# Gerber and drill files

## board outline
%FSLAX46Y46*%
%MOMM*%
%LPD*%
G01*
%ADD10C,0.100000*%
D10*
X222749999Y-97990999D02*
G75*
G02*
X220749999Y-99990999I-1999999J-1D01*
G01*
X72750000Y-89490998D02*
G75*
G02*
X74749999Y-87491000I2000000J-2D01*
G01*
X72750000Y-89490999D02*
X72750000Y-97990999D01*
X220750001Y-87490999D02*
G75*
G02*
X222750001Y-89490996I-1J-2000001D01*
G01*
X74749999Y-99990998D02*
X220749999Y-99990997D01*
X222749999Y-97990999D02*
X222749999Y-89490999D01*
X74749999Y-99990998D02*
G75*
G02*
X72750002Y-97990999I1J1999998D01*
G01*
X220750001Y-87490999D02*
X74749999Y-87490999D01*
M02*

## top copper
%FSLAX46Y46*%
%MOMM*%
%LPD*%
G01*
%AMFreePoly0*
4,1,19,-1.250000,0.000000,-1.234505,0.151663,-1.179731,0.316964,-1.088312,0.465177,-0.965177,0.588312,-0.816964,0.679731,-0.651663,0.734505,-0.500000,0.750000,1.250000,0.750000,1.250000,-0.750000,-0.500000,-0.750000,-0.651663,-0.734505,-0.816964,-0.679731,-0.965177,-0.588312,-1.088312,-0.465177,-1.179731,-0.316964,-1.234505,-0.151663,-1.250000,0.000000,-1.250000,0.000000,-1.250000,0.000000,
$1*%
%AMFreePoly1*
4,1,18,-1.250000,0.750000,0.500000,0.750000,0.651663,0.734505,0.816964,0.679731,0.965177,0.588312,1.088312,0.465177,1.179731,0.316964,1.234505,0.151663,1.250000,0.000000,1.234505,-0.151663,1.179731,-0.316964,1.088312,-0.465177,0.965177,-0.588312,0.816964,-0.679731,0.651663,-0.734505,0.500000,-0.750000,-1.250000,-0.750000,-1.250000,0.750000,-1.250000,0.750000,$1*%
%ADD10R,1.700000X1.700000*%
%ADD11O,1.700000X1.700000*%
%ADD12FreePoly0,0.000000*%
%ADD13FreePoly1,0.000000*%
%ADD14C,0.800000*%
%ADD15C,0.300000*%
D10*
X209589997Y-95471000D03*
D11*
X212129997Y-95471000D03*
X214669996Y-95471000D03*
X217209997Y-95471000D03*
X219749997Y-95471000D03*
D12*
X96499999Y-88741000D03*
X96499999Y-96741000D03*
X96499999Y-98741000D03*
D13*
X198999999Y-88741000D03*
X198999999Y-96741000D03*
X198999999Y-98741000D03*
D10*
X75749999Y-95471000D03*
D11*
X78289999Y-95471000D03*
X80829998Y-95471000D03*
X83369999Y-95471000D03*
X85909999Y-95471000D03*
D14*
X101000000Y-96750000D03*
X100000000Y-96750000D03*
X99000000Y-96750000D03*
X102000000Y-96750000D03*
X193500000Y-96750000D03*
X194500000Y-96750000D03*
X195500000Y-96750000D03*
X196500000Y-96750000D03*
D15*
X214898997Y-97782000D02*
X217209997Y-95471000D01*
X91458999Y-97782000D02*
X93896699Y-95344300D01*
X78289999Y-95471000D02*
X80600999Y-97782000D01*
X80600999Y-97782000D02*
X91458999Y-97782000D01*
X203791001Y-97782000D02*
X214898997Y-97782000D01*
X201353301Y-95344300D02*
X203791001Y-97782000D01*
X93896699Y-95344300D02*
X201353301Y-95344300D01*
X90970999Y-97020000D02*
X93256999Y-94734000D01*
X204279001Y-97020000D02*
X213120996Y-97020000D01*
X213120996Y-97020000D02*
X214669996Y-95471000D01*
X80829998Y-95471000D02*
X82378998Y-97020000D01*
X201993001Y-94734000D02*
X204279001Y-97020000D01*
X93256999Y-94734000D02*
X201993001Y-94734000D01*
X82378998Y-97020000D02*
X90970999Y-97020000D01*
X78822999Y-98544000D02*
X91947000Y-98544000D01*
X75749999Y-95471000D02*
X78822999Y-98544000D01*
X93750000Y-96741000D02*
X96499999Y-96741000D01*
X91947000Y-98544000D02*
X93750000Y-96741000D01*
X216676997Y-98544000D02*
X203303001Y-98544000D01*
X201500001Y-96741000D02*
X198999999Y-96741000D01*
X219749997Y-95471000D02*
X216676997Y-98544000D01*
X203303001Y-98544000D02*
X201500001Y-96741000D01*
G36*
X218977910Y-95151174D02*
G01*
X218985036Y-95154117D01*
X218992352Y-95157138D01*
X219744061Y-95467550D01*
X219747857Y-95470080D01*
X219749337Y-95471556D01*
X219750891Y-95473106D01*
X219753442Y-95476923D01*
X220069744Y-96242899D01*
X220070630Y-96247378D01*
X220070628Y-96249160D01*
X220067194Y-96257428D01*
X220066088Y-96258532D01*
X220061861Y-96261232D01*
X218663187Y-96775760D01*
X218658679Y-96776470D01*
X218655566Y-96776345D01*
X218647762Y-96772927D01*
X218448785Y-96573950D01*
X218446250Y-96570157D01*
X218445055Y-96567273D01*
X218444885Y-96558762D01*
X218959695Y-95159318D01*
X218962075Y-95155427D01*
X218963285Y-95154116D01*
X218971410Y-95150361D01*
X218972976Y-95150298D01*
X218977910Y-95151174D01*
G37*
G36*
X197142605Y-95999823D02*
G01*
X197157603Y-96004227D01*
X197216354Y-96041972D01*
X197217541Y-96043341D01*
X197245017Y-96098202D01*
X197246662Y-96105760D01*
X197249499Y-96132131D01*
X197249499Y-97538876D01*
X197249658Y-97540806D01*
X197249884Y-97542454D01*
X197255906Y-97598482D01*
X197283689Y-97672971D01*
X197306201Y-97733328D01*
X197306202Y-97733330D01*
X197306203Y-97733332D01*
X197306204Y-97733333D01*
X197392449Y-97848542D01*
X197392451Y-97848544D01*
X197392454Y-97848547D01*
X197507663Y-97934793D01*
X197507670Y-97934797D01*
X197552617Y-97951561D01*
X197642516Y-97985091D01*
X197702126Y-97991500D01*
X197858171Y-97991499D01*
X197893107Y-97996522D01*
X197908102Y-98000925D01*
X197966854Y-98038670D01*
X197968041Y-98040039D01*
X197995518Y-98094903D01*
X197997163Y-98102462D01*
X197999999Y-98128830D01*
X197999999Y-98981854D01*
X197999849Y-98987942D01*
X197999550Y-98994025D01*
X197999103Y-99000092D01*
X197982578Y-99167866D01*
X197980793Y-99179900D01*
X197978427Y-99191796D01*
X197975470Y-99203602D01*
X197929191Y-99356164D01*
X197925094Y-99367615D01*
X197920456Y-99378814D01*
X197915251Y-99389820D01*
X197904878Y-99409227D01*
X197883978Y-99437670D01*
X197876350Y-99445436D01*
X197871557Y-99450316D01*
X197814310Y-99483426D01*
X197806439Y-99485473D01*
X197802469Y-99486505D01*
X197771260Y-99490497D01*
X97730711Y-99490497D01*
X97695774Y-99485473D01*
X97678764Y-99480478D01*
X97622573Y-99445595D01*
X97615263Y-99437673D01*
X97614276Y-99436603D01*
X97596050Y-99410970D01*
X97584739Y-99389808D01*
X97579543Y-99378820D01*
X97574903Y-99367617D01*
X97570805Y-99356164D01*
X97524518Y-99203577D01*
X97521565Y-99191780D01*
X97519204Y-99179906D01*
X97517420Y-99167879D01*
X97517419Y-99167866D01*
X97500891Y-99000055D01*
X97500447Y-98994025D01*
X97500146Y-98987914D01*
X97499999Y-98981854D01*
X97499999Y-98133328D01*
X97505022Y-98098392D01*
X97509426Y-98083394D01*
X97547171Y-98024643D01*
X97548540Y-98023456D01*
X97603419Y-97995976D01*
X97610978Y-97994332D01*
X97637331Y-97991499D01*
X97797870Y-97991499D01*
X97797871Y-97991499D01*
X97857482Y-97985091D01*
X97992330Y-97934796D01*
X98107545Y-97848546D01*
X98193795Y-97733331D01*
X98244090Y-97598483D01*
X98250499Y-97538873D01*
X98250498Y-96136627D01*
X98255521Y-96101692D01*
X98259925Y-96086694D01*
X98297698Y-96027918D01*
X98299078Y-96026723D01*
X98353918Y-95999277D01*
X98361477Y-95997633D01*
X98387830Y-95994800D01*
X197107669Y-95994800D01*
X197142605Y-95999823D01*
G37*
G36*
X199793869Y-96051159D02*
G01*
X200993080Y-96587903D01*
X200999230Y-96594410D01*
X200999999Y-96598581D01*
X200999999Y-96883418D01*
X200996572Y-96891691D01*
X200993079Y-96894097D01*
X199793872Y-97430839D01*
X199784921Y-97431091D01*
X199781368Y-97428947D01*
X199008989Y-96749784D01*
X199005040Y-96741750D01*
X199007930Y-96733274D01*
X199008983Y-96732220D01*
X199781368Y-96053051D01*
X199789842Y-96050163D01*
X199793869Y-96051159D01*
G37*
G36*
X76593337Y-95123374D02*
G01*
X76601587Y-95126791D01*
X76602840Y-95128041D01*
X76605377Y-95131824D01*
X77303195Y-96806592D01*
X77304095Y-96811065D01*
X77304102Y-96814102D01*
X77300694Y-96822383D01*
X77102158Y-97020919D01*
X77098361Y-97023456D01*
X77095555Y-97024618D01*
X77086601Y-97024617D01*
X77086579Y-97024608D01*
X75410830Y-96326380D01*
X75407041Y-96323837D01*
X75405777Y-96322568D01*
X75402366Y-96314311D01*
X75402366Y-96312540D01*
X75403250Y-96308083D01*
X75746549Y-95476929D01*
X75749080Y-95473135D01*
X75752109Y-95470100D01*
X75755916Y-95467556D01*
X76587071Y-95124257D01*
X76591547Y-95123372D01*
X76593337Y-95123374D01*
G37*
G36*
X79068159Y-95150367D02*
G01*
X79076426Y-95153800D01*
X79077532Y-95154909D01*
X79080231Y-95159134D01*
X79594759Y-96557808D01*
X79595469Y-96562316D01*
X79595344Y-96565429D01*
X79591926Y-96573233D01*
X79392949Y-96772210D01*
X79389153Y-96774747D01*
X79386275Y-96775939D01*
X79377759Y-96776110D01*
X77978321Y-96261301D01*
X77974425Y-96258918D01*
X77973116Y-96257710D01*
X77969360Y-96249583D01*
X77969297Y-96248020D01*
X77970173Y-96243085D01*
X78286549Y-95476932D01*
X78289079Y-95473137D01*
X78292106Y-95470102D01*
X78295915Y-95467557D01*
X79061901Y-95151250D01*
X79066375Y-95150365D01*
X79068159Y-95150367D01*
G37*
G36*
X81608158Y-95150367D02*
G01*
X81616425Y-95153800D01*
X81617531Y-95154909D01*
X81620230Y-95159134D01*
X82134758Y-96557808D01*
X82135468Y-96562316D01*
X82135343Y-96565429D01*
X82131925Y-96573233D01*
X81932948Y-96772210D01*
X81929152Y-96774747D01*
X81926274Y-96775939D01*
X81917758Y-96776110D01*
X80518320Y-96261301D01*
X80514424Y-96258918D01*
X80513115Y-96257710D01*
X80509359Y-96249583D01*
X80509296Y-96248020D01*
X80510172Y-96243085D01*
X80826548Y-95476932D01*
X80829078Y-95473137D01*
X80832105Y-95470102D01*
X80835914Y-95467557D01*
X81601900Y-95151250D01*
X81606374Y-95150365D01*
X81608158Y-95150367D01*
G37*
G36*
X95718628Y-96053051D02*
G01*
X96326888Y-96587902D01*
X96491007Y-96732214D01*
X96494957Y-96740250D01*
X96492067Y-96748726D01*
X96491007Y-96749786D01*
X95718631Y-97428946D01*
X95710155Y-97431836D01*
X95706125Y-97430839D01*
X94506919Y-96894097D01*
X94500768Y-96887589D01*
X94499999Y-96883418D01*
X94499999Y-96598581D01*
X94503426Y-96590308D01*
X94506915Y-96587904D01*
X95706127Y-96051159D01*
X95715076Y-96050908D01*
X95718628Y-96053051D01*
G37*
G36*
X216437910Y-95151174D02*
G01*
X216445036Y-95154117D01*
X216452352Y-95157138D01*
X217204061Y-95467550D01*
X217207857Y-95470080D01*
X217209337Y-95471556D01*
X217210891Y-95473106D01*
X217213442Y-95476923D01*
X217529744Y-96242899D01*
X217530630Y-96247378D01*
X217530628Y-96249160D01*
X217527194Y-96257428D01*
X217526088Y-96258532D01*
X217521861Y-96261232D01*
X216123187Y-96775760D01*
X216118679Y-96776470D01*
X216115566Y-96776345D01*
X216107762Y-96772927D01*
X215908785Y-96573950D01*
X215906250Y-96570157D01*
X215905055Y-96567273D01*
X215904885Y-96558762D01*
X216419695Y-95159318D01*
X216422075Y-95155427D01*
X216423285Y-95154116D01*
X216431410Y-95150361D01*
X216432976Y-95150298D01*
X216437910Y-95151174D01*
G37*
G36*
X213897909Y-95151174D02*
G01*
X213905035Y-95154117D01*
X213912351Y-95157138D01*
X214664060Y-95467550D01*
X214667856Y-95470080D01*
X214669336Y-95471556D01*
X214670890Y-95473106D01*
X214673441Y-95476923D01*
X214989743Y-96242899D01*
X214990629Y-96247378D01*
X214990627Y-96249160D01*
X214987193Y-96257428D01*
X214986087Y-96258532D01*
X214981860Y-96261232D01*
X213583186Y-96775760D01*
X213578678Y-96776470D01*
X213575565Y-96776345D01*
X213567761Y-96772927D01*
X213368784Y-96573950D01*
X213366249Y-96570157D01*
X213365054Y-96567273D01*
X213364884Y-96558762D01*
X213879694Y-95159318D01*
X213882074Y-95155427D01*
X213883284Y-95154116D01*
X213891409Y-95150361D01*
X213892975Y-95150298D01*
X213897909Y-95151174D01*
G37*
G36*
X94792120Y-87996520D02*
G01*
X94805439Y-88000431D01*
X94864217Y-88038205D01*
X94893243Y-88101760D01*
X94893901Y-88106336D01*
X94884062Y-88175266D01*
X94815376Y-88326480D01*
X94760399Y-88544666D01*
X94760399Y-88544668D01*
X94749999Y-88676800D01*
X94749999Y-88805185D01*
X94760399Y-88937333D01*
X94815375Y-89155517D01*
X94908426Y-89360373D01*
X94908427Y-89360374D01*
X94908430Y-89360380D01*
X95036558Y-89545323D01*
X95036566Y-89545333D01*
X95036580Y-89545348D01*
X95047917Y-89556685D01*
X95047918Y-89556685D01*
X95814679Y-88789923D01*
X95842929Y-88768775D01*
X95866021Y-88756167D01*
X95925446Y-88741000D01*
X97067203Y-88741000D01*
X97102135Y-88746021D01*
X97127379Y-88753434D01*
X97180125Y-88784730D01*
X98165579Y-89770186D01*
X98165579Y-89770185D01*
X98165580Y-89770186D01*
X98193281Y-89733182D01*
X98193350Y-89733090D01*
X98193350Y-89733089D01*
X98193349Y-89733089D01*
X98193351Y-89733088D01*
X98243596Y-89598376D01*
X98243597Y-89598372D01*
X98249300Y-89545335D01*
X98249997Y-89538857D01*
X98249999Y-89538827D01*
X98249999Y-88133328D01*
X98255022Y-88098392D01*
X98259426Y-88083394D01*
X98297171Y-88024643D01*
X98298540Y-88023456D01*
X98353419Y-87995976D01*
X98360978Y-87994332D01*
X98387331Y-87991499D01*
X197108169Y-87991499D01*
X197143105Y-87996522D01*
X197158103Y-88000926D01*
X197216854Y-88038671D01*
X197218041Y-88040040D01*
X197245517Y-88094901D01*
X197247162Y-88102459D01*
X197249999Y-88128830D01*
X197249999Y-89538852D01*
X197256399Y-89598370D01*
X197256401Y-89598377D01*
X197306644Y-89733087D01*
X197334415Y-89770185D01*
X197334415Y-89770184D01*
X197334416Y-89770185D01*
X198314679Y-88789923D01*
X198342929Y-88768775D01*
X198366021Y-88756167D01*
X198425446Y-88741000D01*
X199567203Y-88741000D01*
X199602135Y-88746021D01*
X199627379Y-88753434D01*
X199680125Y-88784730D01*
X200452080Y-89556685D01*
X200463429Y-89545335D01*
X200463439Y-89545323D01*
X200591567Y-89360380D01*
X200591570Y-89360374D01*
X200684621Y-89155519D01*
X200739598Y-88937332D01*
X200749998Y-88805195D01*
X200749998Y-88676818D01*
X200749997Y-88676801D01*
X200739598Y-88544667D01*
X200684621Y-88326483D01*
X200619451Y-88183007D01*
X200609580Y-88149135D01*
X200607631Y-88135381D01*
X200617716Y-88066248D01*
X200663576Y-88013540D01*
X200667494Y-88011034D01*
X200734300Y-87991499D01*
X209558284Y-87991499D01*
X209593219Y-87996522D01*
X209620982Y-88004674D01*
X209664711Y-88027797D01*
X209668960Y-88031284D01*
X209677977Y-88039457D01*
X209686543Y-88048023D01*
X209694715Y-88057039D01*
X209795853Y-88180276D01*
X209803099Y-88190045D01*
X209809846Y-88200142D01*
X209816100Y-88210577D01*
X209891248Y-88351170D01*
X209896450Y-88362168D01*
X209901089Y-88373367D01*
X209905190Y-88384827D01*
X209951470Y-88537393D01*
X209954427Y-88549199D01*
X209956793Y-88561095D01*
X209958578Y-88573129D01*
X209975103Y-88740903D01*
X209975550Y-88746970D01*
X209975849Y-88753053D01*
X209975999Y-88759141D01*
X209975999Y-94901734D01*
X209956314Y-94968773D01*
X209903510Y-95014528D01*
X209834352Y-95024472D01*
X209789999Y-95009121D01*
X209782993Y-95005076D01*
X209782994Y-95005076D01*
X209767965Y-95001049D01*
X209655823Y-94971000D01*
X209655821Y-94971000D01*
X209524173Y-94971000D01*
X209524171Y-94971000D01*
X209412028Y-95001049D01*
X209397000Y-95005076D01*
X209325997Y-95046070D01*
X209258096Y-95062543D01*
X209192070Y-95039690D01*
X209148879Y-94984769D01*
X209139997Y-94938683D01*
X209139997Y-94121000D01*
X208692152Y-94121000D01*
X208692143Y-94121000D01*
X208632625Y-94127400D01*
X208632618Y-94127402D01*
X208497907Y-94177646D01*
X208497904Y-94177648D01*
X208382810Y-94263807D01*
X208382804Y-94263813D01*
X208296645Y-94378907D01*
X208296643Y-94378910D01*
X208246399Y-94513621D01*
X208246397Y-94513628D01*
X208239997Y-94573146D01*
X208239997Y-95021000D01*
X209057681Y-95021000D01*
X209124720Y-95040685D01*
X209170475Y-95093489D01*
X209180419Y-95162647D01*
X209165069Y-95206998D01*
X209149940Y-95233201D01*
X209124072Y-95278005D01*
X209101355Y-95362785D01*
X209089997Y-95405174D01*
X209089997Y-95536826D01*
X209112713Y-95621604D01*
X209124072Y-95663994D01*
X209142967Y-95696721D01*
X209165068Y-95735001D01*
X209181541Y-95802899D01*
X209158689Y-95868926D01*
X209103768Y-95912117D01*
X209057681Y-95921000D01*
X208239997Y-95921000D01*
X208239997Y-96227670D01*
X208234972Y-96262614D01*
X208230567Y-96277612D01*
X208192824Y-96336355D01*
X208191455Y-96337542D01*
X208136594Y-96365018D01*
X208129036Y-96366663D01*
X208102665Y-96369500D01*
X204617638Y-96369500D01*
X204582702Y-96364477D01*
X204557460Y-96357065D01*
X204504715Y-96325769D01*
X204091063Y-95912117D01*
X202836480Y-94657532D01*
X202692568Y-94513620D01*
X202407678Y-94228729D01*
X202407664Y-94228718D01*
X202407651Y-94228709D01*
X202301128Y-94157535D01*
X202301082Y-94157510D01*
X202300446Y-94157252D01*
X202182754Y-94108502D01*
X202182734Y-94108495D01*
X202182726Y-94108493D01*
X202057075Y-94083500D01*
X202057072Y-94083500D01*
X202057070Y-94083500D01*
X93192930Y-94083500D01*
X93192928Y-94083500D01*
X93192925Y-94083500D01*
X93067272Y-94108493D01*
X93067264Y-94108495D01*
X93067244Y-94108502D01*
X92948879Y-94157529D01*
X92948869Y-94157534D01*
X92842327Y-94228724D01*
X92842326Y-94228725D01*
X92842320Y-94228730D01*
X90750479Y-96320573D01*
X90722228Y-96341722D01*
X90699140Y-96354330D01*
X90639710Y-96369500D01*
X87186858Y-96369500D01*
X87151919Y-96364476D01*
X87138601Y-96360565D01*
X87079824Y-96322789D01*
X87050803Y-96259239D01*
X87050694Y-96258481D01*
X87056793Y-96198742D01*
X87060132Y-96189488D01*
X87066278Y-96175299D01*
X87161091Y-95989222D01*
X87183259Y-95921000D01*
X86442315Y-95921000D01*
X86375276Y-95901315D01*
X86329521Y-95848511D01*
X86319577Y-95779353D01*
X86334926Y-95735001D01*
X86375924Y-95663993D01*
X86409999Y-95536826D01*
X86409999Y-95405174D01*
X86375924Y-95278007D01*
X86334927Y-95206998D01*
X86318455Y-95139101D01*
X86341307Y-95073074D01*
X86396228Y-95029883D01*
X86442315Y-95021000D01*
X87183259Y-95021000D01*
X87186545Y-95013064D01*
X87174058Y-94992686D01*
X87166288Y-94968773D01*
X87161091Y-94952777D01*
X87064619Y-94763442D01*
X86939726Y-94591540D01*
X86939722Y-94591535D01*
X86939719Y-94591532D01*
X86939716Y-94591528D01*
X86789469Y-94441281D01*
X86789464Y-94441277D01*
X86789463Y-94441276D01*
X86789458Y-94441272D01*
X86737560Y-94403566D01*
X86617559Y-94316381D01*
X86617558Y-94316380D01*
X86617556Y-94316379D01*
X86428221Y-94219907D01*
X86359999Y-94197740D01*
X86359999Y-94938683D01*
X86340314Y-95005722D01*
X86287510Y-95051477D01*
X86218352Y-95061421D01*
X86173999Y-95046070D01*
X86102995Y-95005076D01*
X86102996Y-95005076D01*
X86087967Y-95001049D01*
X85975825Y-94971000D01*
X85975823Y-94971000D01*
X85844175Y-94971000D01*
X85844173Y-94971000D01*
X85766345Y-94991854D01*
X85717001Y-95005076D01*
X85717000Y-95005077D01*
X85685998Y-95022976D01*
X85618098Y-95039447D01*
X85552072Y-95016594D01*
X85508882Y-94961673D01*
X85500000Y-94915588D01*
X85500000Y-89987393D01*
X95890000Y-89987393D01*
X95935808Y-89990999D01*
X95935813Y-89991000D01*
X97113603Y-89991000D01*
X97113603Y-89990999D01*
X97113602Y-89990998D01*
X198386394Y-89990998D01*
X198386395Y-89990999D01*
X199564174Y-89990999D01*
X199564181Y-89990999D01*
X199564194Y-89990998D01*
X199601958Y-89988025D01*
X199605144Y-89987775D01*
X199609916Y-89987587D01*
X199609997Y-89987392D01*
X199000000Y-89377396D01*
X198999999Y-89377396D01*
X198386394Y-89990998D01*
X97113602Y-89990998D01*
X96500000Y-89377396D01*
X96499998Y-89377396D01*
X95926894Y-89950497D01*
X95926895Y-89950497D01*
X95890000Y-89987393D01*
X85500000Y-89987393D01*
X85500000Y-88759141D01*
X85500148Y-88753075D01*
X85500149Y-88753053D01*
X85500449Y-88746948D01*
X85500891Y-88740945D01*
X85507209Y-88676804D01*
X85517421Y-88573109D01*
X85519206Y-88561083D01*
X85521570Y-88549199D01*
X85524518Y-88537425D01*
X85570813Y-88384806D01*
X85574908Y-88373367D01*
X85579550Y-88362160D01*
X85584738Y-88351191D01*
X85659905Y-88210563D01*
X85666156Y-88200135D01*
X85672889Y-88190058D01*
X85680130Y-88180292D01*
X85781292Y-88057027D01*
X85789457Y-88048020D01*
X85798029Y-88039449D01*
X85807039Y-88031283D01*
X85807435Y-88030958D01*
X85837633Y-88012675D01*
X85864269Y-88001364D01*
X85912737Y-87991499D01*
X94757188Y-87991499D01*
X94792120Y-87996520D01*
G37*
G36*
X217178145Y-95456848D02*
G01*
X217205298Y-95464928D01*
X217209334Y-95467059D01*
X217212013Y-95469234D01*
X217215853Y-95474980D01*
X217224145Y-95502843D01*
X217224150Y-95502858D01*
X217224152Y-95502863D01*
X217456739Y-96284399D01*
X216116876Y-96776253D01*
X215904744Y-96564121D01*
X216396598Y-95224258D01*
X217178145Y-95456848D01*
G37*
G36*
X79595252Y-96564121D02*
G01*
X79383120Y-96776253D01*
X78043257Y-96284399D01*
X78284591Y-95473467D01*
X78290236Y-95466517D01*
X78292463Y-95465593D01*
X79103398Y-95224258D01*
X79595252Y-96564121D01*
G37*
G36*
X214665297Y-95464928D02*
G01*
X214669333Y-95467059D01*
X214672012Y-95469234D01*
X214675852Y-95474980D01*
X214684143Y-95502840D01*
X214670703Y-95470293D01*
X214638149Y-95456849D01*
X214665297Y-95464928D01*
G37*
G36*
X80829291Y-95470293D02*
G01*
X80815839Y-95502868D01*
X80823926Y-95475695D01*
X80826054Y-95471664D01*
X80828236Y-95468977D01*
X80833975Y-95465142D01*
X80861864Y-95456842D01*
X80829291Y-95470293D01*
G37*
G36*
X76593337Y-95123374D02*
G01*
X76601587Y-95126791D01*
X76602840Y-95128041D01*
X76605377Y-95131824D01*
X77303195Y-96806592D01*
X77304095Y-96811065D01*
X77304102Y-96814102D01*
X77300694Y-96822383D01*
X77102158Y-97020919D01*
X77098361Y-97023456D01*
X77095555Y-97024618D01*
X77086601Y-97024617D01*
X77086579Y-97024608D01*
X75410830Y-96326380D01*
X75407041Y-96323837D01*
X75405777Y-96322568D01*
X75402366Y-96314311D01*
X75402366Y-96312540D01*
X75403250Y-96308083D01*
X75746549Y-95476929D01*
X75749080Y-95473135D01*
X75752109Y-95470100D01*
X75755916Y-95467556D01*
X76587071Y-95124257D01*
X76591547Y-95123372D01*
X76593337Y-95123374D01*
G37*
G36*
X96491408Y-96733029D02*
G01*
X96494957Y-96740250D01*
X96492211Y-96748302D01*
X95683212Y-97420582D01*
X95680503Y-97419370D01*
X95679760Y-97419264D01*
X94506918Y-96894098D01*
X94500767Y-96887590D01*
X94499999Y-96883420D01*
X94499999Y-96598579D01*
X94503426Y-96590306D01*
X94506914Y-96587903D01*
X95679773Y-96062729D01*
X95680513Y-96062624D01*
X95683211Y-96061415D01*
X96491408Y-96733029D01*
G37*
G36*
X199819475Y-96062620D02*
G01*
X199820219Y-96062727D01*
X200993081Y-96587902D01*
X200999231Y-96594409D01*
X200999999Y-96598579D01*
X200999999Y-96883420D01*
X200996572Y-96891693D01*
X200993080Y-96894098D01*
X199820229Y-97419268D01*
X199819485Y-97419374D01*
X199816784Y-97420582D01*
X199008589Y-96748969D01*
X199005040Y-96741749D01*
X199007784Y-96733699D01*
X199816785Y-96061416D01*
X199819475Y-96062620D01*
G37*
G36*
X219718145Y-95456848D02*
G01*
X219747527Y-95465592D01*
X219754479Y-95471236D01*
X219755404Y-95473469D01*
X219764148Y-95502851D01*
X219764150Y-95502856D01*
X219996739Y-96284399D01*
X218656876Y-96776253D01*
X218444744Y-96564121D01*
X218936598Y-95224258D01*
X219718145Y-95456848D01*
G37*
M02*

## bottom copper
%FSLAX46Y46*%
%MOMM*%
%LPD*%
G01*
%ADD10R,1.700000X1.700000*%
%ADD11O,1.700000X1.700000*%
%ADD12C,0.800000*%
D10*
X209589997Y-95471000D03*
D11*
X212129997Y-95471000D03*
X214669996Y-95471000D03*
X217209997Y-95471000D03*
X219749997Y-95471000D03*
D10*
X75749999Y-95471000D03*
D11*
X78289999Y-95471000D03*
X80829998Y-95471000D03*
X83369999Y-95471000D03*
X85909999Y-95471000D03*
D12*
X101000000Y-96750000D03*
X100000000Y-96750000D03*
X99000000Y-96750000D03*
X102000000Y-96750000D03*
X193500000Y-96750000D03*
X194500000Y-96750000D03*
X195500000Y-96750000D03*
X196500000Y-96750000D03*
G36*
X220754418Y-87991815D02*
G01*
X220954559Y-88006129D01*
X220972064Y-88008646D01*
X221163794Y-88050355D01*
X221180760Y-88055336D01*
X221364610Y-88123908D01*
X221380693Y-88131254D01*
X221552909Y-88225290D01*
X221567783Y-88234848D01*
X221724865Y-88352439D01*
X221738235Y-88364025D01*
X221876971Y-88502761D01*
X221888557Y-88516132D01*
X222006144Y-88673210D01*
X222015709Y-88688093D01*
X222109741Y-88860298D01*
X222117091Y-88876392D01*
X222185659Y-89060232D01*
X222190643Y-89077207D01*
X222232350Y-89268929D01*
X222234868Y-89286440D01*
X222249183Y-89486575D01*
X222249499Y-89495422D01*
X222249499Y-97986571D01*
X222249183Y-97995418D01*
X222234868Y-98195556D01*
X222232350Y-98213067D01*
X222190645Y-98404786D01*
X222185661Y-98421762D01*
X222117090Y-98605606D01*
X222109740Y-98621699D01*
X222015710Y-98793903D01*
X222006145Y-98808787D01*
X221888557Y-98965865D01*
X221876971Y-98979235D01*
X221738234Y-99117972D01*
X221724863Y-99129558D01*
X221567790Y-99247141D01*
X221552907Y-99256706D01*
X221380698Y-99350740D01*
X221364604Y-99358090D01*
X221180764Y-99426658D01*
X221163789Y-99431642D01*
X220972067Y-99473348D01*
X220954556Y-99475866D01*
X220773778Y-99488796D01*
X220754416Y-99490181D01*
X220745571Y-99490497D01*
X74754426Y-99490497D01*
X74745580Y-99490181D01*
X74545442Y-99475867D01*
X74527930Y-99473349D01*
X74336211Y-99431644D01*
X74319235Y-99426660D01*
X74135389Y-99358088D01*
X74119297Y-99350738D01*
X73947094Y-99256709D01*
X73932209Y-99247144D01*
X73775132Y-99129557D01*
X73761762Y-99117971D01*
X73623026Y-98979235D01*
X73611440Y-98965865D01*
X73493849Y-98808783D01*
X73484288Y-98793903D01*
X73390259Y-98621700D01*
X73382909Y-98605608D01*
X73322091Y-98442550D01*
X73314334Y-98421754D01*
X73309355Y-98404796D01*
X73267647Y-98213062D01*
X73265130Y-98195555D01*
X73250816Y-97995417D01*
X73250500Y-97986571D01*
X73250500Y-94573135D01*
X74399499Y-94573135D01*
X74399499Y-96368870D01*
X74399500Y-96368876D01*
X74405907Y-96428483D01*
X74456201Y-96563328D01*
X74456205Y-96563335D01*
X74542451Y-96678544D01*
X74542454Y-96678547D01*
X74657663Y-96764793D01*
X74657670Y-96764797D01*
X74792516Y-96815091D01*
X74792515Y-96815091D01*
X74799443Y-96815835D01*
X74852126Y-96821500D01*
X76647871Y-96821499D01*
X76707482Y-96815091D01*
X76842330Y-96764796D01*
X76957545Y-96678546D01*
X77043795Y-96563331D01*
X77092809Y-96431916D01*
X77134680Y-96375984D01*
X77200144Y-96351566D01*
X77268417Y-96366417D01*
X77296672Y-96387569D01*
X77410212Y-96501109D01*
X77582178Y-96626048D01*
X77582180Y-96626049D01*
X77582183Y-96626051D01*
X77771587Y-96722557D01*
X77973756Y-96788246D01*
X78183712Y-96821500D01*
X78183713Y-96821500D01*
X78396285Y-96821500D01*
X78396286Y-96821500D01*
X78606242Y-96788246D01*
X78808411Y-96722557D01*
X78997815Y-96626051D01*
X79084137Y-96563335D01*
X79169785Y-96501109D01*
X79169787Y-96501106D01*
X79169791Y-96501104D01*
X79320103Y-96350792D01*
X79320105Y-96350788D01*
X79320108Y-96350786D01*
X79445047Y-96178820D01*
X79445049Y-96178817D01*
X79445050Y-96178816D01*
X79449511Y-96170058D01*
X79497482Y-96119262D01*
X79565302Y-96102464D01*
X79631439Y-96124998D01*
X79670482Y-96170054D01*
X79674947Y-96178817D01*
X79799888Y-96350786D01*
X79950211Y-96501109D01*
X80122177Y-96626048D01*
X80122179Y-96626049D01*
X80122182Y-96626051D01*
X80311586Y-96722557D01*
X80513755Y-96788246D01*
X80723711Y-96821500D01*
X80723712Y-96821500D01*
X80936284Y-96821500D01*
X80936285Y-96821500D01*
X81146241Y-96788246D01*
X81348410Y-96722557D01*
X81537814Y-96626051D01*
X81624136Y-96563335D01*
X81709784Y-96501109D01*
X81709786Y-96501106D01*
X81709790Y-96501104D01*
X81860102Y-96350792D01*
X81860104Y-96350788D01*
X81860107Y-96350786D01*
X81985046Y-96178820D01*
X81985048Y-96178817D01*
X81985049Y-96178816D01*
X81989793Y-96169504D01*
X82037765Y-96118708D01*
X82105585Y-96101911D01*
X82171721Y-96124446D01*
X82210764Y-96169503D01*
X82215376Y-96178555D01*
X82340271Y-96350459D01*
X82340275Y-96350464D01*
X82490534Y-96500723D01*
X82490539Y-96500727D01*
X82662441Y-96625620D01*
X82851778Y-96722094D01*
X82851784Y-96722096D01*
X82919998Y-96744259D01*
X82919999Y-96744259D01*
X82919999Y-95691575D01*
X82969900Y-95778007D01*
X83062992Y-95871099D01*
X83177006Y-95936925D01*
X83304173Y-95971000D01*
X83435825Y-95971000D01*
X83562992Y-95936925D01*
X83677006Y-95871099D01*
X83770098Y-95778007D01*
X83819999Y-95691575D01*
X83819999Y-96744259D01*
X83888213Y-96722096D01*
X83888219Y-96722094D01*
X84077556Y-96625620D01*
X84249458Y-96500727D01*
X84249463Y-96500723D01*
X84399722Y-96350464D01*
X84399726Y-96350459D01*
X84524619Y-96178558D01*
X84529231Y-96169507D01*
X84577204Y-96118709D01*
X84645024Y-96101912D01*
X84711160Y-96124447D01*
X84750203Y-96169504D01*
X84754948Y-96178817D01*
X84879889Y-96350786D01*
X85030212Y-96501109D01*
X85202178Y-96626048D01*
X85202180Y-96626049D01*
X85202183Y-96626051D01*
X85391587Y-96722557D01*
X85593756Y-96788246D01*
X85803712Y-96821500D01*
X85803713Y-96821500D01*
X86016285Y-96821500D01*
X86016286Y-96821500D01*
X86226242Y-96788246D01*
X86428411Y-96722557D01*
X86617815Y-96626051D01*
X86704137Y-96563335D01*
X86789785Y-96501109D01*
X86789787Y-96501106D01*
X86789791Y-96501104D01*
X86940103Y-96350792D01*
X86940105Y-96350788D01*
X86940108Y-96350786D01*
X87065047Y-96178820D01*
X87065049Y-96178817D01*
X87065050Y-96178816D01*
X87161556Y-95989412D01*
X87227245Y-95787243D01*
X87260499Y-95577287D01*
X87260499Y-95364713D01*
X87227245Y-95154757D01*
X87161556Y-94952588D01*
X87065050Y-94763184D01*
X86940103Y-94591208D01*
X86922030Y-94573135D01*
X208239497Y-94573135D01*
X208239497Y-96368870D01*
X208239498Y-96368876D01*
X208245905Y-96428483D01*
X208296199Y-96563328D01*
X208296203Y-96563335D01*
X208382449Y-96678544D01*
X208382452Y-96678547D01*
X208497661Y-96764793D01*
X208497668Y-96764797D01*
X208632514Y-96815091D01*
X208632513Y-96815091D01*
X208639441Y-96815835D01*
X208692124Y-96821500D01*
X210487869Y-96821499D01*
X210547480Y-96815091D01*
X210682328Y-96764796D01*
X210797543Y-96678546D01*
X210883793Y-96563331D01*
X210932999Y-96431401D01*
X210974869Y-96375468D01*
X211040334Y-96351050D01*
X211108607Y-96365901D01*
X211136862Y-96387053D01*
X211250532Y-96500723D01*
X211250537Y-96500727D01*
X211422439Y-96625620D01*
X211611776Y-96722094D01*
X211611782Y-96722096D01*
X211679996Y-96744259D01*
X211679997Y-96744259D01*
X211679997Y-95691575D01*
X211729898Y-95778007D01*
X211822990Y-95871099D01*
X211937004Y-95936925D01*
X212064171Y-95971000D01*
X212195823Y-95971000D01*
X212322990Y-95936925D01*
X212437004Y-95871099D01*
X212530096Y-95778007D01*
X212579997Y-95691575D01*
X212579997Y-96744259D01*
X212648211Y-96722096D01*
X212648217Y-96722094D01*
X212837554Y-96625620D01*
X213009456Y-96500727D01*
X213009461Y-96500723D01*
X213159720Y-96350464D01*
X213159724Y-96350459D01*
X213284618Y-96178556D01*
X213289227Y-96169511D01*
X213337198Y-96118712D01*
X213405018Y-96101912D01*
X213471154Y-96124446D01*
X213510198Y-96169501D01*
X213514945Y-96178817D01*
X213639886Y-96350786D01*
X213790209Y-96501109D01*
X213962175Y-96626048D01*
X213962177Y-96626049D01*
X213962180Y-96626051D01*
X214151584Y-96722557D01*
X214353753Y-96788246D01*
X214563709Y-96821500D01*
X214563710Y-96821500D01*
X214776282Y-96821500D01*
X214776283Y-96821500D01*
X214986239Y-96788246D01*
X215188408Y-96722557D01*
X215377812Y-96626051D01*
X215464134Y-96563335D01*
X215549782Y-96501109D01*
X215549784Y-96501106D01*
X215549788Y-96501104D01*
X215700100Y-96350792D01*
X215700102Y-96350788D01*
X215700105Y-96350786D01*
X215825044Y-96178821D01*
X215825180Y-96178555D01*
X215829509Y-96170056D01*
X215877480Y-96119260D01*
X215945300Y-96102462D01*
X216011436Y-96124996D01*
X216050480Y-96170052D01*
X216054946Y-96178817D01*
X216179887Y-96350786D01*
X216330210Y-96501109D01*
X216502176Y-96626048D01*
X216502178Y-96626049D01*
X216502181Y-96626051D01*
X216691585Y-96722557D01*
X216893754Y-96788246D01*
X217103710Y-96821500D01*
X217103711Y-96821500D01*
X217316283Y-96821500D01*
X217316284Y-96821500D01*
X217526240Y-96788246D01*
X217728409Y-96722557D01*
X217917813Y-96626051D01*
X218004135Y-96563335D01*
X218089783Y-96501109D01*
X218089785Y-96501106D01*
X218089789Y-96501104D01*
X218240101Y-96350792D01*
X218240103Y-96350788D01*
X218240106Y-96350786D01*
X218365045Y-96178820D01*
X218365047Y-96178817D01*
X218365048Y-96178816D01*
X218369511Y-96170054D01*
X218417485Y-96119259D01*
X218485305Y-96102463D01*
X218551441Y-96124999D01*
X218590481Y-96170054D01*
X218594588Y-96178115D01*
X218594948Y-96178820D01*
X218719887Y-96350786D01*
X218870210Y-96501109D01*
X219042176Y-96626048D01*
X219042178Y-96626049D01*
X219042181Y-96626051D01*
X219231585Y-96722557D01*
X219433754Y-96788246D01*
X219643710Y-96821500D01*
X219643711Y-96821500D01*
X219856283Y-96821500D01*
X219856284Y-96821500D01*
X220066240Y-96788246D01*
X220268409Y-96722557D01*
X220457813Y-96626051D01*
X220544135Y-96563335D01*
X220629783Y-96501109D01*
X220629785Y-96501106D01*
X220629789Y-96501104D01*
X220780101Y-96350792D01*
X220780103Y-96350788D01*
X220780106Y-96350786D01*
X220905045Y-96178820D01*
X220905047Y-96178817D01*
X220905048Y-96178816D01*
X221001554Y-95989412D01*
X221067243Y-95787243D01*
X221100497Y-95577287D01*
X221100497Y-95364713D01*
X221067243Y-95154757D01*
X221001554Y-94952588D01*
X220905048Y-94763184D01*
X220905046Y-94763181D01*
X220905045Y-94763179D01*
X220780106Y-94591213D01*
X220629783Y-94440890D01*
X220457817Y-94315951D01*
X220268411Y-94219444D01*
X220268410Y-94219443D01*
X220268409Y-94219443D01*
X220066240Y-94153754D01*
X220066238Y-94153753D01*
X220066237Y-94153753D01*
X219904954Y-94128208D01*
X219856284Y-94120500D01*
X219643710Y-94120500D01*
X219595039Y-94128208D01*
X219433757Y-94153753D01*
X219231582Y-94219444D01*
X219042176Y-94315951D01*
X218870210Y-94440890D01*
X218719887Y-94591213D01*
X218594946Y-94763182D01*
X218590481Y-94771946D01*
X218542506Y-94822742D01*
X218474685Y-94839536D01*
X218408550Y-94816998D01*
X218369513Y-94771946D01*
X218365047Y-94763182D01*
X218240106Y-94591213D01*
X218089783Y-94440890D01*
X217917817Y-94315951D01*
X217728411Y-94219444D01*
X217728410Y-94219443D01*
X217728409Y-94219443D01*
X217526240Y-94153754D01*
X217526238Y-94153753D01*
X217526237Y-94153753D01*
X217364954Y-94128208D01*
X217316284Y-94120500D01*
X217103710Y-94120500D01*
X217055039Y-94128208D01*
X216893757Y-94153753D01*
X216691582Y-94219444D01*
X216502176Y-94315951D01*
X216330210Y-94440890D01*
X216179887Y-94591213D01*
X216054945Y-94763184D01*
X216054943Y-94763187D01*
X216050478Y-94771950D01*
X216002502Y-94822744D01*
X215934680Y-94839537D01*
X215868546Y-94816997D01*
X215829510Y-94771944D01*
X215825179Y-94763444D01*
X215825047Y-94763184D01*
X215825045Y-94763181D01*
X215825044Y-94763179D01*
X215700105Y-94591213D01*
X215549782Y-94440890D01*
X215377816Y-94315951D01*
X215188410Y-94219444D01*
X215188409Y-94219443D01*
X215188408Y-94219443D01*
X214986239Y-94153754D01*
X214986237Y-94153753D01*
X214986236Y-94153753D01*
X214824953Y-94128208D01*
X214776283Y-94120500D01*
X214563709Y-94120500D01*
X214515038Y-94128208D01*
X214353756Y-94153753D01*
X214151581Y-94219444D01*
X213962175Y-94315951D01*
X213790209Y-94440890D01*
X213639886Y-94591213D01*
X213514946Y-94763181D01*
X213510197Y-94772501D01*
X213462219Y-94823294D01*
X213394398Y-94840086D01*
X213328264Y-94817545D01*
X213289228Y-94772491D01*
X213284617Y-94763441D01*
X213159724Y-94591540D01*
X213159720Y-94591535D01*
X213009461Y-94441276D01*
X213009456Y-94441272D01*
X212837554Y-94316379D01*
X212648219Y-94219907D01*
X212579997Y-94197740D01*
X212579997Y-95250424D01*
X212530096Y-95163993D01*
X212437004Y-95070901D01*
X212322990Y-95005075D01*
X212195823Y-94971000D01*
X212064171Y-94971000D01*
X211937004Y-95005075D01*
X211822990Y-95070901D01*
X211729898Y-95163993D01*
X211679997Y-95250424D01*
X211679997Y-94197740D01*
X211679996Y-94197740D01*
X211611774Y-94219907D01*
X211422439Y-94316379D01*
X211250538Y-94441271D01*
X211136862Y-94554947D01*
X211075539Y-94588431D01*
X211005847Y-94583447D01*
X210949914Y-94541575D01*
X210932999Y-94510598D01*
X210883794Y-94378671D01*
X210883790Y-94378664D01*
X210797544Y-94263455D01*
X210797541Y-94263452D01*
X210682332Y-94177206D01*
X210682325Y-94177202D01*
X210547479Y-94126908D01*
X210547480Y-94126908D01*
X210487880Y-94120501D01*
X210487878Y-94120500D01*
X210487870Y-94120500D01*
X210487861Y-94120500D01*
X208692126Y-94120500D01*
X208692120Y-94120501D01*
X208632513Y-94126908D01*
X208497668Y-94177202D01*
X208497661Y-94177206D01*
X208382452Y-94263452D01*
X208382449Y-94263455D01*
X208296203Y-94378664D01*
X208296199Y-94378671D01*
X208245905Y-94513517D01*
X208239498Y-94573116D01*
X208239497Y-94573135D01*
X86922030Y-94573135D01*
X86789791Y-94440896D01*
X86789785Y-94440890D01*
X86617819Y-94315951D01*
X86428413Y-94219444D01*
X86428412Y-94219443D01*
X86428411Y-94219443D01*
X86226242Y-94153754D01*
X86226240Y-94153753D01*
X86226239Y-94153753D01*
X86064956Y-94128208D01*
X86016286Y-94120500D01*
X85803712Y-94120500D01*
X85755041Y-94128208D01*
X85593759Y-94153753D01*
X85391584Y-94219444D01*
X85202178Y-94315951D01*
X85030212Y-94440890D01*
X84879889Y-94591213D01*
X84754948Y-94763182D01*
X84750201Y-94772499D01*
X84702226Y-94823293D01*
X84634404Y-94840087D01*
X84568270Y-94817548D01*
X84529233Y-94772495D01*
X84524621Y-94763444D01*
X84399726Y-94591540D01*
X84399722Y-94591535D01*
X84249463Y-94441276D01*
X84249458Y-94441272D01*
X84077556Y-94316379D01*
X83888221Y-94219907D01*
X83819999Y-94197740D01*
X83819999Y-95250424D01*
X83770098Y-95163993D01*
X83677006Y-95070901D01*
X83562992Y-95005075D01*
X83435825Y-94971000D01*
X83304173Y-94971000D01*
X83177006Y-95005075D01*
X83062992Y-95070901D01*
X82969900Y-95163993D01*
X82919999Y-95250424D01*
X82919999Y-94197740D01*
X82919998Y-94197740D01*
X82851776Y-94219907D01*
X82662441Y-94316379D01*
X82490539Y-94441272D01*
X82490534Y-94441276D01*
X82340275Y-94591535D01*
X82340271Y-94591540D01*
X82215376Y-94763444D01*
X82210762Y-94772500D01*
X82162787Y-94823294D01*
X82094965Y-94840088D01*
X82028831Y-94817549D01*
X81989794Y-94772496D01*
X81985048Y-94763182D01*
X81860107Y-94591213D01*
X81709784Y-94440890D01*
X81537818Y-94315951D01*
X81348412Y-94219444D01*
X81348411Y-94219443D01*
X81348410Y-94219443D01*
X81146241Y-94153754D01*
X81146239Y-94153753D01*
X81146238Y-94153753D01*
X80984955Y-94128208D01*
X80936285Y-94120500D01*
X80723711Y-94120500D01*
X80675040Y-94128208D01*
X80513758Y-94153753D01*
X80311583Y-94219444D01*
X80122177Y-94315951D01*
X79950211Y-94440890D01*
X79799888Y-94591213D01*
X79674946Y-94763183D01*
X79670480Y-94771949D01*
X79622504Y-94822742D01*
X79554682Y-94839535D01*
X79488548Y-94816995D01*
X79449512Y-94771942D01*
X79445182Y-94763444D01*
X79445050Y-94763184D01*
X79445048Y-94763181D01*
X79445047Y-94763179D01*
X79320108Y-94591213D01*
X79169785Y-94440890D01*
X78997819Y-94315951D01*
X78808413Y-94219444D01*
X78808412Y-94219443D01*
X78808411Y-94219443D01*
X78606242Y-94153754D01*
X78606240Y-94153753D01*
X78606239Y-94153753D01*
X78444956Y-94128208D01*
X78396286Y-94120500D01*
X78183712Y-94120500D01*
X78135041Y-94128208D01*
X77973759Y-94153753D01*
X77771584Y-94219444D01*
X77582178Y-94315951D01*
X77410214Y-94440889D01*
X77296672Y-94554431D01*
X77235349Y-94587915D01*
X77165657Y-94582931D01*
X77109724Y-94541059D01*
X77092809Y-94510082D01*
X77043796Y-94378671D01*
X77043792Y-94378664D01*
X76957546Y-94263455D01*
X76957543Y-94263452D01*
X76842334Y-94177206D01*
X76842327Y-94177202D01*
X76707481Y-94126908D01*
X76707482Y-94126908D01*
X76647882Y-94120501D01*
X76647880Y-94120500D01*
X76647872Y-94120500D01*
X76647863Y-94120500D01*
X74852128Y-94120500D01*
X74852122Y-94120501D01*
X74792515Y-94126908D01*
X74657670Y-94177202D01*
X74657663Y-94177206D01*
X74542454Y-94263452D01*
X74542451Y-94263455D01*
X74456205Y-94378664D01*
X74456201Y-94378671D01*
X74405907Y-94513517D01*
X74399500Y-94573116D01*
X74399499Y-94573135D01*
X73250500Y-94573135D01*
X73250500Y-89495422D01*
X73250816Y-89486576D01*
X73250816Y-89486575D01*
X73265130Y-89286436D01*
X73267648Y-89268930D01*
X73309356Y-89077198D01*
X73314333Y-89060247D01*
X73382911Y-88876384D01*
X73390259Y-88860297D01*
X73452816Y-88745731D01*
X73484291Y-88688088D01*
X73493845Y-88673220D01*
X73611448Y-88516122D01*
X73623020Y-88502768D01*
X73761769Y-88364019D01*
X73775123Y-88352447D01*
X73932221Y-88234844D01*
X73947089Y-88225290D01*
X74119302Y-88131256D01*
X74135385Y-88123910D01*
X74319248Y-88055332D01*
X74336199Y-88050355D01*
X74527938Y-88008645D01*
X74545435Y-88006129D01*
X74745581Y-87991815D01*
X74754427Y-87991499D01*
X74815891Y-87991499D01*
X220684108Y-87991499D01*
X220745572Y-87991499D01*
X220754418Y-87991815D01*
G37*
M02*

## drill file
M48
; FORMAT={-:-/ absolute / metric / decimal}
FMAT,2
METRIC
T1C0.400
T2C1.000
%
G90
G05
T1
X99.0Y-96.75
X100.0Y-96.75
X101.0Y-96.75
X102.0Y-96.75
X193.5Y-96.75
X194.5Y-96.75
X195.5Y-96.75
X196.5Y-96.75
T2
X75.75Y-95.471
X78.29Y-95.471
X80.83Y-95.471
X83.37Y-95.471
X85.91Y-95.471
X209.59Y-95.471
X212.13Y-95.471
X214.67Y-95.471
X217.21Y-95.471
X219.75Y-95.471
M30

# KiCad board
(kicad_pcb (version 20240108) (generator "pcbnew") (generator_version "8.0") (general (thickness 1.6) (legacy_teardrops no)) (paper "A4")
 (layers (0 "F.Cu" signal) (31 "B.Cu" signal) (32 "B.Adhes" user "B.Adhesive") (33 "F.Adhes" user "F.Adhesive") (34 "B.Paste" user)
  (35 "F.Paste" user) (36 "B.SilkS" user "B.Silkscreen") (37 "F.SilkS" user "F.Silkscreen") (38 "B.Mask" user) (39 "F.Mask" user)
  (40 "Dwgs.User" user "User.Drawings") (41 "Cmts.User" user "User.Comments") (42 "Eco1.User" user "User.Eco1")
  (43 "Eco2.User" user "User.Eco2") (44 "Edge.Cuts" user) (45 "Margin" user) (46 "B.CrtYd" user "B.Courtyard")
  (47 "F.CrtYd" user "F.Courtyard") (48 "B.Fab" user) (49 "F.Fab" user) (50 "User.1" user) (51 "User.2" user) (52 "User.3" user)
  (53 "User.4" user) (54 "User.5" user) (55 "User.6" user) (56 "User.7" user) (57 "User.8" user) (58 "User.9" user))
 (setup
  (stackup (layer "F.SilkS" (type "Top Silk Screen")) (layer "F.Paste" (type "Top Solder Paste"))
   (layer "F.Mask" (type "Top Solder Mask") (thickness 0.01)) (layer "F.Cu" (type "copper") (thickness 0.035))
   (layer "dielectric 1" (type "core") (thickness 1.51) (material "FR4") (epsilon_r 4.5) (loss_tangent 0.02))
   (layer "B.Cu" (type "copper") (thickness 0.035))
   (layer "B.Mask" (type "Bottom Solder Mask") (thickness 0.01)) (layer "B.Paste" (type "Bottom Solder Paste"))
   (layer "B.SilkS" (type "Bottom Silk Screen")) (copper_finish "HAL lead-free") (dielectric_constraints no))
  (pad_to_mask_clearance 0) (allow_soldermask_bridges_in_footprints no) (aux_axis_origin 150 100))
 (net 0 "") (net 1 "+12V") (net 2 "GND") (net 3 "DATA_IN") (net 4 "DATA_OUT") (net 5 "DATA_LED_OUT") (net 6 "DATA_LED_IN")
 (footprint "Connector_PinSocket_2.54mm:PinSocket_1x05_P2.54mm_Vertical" (layer "F.Cu") (at 209.589997 95.471 90)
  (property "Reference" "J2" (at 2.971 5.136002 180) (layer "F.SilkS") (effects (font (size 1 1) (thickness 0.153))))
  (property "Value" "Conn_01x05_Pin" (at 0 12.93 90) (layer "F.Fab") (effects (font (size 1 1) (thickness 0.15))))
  (pad "1" thru_hole rect (at 0 0 90) (size 1.7 1.7) (drill 1) (layers "*.Cu" "*.Mask") (remove_unused_layers no) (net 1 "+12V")
   (teardrops (best_length_ratio 0.5) (max_length 1) (best_width_ratio 1) (max_width 2) (curve_points 0) (filter_ratio 0.9) (enabled yes)
    (allow_two_segments yes) (prefer_zone_connections yes)))
  (pad "2" thru_hole oval (at 0 2.54 90) (size 1.7 1.7) (drill 1) (layers "*.Cu" "*.Mask") (remove_unused_layers no) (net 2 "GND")
   (teardrops (best_length_ratio 0.5) (max_length 1) (best_width_ratio 1) (max_width 2) (curve_points 0) (filter_ratio 0.9) (enabled yes)
    (allow_two_segments yes) (prefer_zone_connections yes)))
  (pad "3" thru_hole oval (at 0 5.079999 90) (size 1.7 1.7) (drill 1) (layers "*.Cu" "*.Mask") (remove_unused_layers no) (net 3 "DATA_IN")
   (teardrops (best_length_ratio 0.5) (max_length 1) (best_width_ratio 1) (max_width 2) (curve_points 0) (filter_ratio 0.9) (enabled yes)
    (allow_two_segments yes) (prefer_zone_connections yes)))
  (pad "4" thru_hole oval (at 0 7.62 90) (size 1.7 1.7) (drill 1) (layers "*.Cu" "*.Mask") (remove_unused_layers no) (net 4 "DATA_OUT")
   (teardrops (best_length_ratio 0.5) (max_length 1) (best_width_ratio 1) (max_width 2) (curve_points 0) (filter_ratio 0.9) (enabled yes)
    (allow_two_segments yes) (prefer_zone_connections yes)))
  (pad "5" thru_hole oval (at 0 10.16 90) (size 1.7 1.7) (drill 1) (layers "*.Cu" "*.Mask") (remove_unused_layers no) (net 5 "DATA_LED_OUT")
   (teardrops (best_length_ratio 0.5) (max_length 1) (best_width_ratio 1) (max_width 2) (curve_points 0) (filter_ratio 0.9) (enabled yes)
    (allow_two_segments yes) (prefer_zone_connections yes))))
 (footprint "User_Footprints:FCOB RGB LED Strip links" (layer "F.Cu") (at 97.749999 93.741)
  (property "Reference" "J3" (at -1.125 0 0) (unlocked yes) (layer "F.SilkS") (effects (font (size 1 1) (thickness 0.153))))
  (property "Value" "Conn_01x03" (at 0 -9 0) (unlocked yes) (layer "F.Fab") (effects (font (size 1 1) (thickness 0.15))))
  (pad "1" smd roundrect (at -1.25 -5) (size 2.5 1.5) (layers "F.Cu" "F.Paste" "F.Mask") (roundrect_rratio 0.5) (chamfer_ratio 0)
   (chamfer top_right bottom_right) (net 1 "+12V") (thermal_bridge_angle 45)
   (teardrops (best_length_ratio 0.5) (max_length 1) (best_width_ratio 1) (max_width 2) (curve_points 0) (filter_ratio 0.9) (enabled yes)
    (allow_two_segments yes) (prefer_zone_connections yes)))
  (pad "2" smd roundrect (at -1.25 3) (size 2.5 1.5) (layers "F.Cu" "F.Paste" "F.Mask") (roundrect_rratio 0.5) (chamfer_ratio 0)
   (chamfer top_right bottom_right) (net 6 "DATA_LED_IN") (thermal_bridge_angle 45)
   (teardrops (best_length_ratio 0.5) (max_length 1) (best_width_ratio 1) (max_width 2) (curve_points 0) (filter_ratio 0.9) (enabled yes)
    (allow_two_segments yes) (prefer_zone_connections yes)))
  (pad "3" smd roundrect (at -1.25 5) (size 2.5 1.5) (layers "F.Cu" "F.Paste" "F.Mask") (roundrect_rratio 0.5) (chamfer_ratio 0)
   (chamfer top_right bottom_right) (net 2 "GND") (thermal_bridge_angle 45)
   (teardrops (best_length_ratio 0.5) (max_length 1) (best_width_ratio 1) (max_width 2) (curve_points 0) (filter_ratio 0.9) (enabled yes)
    (allow_two_segments yes) (prefer_zone_connections yes))))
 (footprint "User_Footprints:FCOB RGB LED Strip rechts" (layer "F.Cu") (at 197.749999 93.741)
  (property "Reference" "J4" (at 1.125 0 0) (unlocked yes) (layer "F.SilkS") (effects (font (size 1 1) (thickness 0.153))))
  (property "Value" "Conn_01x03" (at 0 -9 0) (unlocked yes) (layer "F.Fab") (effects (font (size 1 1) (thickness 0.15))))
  (pad "1" smd roundrect (at 1.25 -5) (size 2.5 1.5) (layers "F.Cu" "F.Paste" "F.Mask") (roundrect_rratio 0.5) (chamfer_ratio 0)
   (chamfer top_left bottom_left) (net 1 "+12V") (thermal_bridge_angle 45)
   (teardrops (best_length_ratio 0.5) (max_length 1) (best_width_ratio 1) (max_width 2) (curve_points 0) (filter_ratio 0.9) (enabled yes)
    (allow_two_segments yes) (prefer_zone_connections yes)))
  (pad "2" smd roundrect (at 1.25 3) (size 2.5 1.5) (layers "F.Cu" "F.Paste" "F.Mask") (roundrect_rratio 0.5) (chamfer_ratio 0)
   (chamfer top_left bottom_left) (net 5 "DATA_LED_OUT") (thermal_bridge_angle 45)
   (teardrops (best_length_ratio 0.5) (max_length 1) (best_width_ratio 1) (max_width 2) (curve_points 0) (filter_ratio 0.9) (enabled yes)
    (allow_two_segments yes) (prefer_zone_connections yes)))
  (pad "3" smd roundrect (at 1.25 5) (size 2.5 1.5) (layers "F.Cu" "F.Paste" "F.Mask") (roundrect_rratio 0.5) (chamfer_ratio 0)
   (chamfer top_left bottom_left) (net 2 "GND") (thermal_bridge_angle 45)
   (teardrops (best_length_ratio 0.5) (max_length 1) (best_width_ratio 1) (max_width 2) (curve_points 0) (filter_ratio 0.9) (enabled yes)
    (allow_two_segments yes) (prefer_zone_connections yes))))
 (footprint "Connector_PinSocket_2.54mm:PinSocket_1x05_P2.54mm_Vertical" (layer "F.Cu") (at 75.749999 95.471 90)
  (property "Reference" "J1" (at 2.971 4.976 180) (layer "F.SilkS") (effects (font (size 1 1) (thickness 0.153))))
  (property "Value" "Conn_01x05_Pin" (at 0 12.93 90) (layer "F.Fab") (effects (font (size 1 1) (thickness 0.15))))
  (pad "1" thru_hole rect (at 0 0 90) (size 1.7 1.7) (drill 1) (layers "*.Cu" "*.Mask") (remove_unused_layers no) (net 6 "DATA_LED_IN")
   (teardrops (best_length_ratio 0.5) (max_length 1) (best_width_ratio 1) (max_width 2) (curve_points 0) (filter_ratio 0.9) (enabled yes)
    (allow_two_segments yes) (prefer_zone_connections yes)))
  (pad "2" thru_hole oval (at 0 2.54 90) (size 1.7 1.7) (drill 1) (layers "*.Cu" "*.Mask") (remove_unused_layers no) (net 4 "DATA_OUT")
   (teardrops (best_length_ratio 0.5) (max_length 1) (best_width_ratio 1) (max_width 2) (curve_points 0) (filter_ratio 0.9) (enabled yes)
    (allow_two_segments yes) (prefer_zone_connections yes)))
  (pad "3" thru_hole oval (at 0 5.079999 90) (size 1.7 1.7) (drill 1) (layers "*.Cu" "*.Mask") (remove_unused_layers no) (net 3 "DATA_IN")
   (teardrops (best_length_ratio 0.5) (max_length 1) (best_width_ratio 1) (max_width 2) (curve_points 0) (filter_ratio 0.9) (enabled yes)
    (allow_two_segments yes) (prefer_zone_connections yes)))
  (pad "4" thru_hole oval (at 0 7.62 90) (size 1.7 1.7) (drill 1) (layers "*.Cu" "*.Mask") (remove_unused_layers no) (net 2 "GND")
   (teardrops (best_length_ratio 0.5) (max_length 1) (best_width_ratio 1) (max_width 2) (curve_points 0) (filter_ratio 0.9) (enabled yes)
    (allow_two_segments yes) (prefer_zone_connections yes)))
  (pad "5" thru_hole oval (at 0 10.16 90) (size 1.7 1.7) (drill 1) (layers "*.Cu" "*.Mask") (remove_unused_layers no) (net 1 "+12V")
   (teardrops (best_length_ratio 0.5) (max_length 1) (best_width_ratio 1) (max_width 2) (curve_points 0) (filter_ratio 0.9) (enabled yes)
    (allow_two_segments yes) (prefer_zone_connections yes))))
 (gr_arc (start 222.749999 97.990999) (mid 222.164212 99.405212) (end 220.749999 99.990997) (stroke (width 0.1) (type default))
  (layer "Edge.Cuts"))
 (gr_arc (start 72.75 89.490998) (mid 73.335786 88.076786) (end 74.749999 87.490999) (stroke (width 0.1) (type default)) (layer "Edge.Cuts"))
 (gr_line (start 72.75 89.490999) (end 72.75 97.990999) (stroke (width 0.1) (type default)) (layer "Edge.Cuts"))
 (gr_arc (start 220.750001 87.490999) (mid 222.164212 88.076785) (end 222.749999 89.490996) (stroke (width 0.1) (type default))
  (layer "Edge.Cuts"))
 (gr_line (start 74.749999 99.990998) (end 220.749999 99.990997) (stroke (width 0.1) (type default)) (layer "Edge.Cuts"))
 (gr_line (start 222.749999 97.990999) (end 222.749999 89.490999) (stroke (width 0.1) (type default)) (layer "Edge.Cuts"))
 (gr_arc (start 74.749999 99.990998) (mid 73.335786 99.405212) (end 72.75 97.990999) (stroke (width 0.1) (type default)) (layer "Edge.Cuts"))
 (gr_line (start 220.750001 87.490999) (end 74.749999 87.490999) (stroke (width 0.1) (type default)) (layer "Edge.Cuts"))
 (segment (start 214.898997 97.782) (end 217.209997 95.471) (width 0.3) (layer "F.Cu") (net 4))
 (segment (start 91.458999 97.782) (end 93.896699 95.3443) (width 0.3) (layer "F.Cu") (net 4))
 (segment (start 78.289999 95.471) (end 80.600999 97.782) (width 0.3) (layer "F.Cu") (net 4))
 (segment (start 80.600999 97.782) (end 91.458999 97.782) (width 0.3) (layer "F.Cu") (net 4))
 (segment (start 203.791001 97.782) (end 214.898997 97.782) (width 0.3) (layer "F.Cu") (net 4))
 (segment (start 201.353301 95.3443) (end 203.791001 97.782) (width 0.3) (layer "F.Cu") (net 4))
 (segment (start 93.896699 95.3443) (end 201.353301 95.3443) (width 0.3) (layer "F.Cu") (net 4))
 (via (at 101 96.75) (size 0.8) (drill 0.4) (layers "F.Cu" "B.Cu") (free yes)
  (teardrops (best_length_ratio 0.5) (max_length 1) (best_width_ratio 1) (max_width 2) (curve_points 0) (filter_ratio 0.9) (enabled yes)
   (allow_two_segments yes) (prefer_zone_connections yes))
  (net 2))
 (via (at 100 96.75) (size 0.8) (drill 0.4) (layers "F.Cu" "B.Cu") (free yes)
  (teardrops (best_length_ratio 0.5) (max_length 1) (best_width_ratio 1) (max_width 2) (curve_points 0) (filter_ratio 0.9) (enabled yes)
   (allow_two_segments yes) (prefer_zone_connections yes))
  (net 2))
 (via (at 99 96.75) (size 0.8) (drill 0.4) (layers "F.Cu" "B.Cu") (free yes)
  (teardrops (best_length_ratio 0.5) (max_length 1) (best_width_ratio 1) (max_width 2) (curve_points 0) (filter_ratio 0.9) (enabled yes)
   (allow_two_segments yes) (prefer_zone_connections yes))
  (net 2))
 (via (at 102 96.75) (size 0.8) (drill 0.4) (layers "F.Cu" "B.Cu") (free yes)
  (teardrops (best_length_ratio 0.5) (max_length 1) (best_width_ratio 1) (max_width 2) (curve_points 0) (filter_ratio 0.9) (enabled yes)
   (allow_two_segments yes) (prefer_zone_connections yes))
  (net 2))
 (via (at 193.5 96.75) (size 0.8) (drill 0.4) (layers "F.Cu" "B.Cu") (free yes)
  (teardrops (best_length_ratio 0.5) (max_length 1) (best_width_ratio 1) (max_width 2) (curve_points 0) (filter_ratio 0.9) (enabled yes)
   (allow_two_segments yes) (prefer_zone_connections yes))
  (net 2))
 (via (at 194.5 96.75) (size 0.8) (drill 0.4) (layers "F.Cu" "B.Cu") (free yes)
  (teardrops (best_length_ratio 0.5) (max_length 1) (best_width_ratio 1) (max_width 2) (curve_points 0) (filter_ratio 0.9) (enabled yes)
   (allow_two_segments yes) (prefer_zone_connections yes))
  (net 2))
 (via (at 195.5 96.75) (size 0.8) (drill 0.4) (layers "F.Cu" "B.Cu") (free yes)
  (teardrops (best_length_ratio 0.5) (max_length 1) (best_width_ratio 1) (max_width 2) (curve_points 0) (filter_ratio 0.9) (enabled yes)
   (allow_two_segments yes) (prefer_zone_connections yes))
  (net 2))
 (via (at 196.5 96.75) (size 0.8) (drill 0.4) (layers "F.Cu" "B.Cu") (free yes)
  (teardrops (best_length_ratio 0.5) (max_length 1) (best_width_ratio 1) (max_width 2) (curve_points 0) (filter_ratio 0.9) (enabled yes)
   (allow_two_segments yes) (prefer_zone_connections yes))
  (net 2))
 (segment (start 90.970999 97.02) (end 93.256999 94.734) (width 0.3) (layer "F.Cu") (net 3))
 (segment (start 204.279001 97.02) (end 213.120996 97.02) (width 0.3) (layer "F.Cu") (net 3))
 (segment (start 213.120996 97.02) (end 214.669996 95.471) (width 0.3) (layer "F.Cu") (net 3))
 (segment (start 80.829998 95.471) (end 82.378998 97.02) (width 0.3) (layer "F.Cu") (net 3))
 (segment (start 201.993001 94.734) (end 204.279001 97.02) (width 0.3) (layer "F.Cu") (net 3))
 (segment (start 93.256999 94.734) (end 201.993001 94.734) (width 0.3) (layer "F.Cu") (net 3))
 (segment (start 82.378998 97.02) (end 90.970999 97.02) (width 0.3) (layer "F.Cu") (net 3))
 (segment (start 78.822999 98.544) (end 91.947 98.544) (width 0.3) (layer "F.Cu") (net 6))
 (segment (start 75.749999 95.471) (end 78.822999 98.544) (width 0.3) (layer "F.Cu") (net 6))
 (segment (start 93.75 96.741) (end 96.499999 96.741) (width 0.3) (layer "F.Cu") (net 6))
 (segment (start 91.947 98.544) (end 93.75 96.741) (width 0.3) (layer "F.Cu") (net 6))
 (segment (start 216.676997 98.544) (end 203.303001 98.544) (width 0.3) (layer "F.Cu") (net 5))
 (segment (start 201.500001 96.741) (end 198.999999 96.741) (width 0.3) (layer "F.Cu") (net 5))
 (segment (start 219.749997 95.471) (end 216.676997 98.544) (width 0.3) (layer "F.Cu") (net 5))
 (segment (start 203.303001 98.544) (end 201.500001 96.741) (width 0.3) (layer "F.Cu") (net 5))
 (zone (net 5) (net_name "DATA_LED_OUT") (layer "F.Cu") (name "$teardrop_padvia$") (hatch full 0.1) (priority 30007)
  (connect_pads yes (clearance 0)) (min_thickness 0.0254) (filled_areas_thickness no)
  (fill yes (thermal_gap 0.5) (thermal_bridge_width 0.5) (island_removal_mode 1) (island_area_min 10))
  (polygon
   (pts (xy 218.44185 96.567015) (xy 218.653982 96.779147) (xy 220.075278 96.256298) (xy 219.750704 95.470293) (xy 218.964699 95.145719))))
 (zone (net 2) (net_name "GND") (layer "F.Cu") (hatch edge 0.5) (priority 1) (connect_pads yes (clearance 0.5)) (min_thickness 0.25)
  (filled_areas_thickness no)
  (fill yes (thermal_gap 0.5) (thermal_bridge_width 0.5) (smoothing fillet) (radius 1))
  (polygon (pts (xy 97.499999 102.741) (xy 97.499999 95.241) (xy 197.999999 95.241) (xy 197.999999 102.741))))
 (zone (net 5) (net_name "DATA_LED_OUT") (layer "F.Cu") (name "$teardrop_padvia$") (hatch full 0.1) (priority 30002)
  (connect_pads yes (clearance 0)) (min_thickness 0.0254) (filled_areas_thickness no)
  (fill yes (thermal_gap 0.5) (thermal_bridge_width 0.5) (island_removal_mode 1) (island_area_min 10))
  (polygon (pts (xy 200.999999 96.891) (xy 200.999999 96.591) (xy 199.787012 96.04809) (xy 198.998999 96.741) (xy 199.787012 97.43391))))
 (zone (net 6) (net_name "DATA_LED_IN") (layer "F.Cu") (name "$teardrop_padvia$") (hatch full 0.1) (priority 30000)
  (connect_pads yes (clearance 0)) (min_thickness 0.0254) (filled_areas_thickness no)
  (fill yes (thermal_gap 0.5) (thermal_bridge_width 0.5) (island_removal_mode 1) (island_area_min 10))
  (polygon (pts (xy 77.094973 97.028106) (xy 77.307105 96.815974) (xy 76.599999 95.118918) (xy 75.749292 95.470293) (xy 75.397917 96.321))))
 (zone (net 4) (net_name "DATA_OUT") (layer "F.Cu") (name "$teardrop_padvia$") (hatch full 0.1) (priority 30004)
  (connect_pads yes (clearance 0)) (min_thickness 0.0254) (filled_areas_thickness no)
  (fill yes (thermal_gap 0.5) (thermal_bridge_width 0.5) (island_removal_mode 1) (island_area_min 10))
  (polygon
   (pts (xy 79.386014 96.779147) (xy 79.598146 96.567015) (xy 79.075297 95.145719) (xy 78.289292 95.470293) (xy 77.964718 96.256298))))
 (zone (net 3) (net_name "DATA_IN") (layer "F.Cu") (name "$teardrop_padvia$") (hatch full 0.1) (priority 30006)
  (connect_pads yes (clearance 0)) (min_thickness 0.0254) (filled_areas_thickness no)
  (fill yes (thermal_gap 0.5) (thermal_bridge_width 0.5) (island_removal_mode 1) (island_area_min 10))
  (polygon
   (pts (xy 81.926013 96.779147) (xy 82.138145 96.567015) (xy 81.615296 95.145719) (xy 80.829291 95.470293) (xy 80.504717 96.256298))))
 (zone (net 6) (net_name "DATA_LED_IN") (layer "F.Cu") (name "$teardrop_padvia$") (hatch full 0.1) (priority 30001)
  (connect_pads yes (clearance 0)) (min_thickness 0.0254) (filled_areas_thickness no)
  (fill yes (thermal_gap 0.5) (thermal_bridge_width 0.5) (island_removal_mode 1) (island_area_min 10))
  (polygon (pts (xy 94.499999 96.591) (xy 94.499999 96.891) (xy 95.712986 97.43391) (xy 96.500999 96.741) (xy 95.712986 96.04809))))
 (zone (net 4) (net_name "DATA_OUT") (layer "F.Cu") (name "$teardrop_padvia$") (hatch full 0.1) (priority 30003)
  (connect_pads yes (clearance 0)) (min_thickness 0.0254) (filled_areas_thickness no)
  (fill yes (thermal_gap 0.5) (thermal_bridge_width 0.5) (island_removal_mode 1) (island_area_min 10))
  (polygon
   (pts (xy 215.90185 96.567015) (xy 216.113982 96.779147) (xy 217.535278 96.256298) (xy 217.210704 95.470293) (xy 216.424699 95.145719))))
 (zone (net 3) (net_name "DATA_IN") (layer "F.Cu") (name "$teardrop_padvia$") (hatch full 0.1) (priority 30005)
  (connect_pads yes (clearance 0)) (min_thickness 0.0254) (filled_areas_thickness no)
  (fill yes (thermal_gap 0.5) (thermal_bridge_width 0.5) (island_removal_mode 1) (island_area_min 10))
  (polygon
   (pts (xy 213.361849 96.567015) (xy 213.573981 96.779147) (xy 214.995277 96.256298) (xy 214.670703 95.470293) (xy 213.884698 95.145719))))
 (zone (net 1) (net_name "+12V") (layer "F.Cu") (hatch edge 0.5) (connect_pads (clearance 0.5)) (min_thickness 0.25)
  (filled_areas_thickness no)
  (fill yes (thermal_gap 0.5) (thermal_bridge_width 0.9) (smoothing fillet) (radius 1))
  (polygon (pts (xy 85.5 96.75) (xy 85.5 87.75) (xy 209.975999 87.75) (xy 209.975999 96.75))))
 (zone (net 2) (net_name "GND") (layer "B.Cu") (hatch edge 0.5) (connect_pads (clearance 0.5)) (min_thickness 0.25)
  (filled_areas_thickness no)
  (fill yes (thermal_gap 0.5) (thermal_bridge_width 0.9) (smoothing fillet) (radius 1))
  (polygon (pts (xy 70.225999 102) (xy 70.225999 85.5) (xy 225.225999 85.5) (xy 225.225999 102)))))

